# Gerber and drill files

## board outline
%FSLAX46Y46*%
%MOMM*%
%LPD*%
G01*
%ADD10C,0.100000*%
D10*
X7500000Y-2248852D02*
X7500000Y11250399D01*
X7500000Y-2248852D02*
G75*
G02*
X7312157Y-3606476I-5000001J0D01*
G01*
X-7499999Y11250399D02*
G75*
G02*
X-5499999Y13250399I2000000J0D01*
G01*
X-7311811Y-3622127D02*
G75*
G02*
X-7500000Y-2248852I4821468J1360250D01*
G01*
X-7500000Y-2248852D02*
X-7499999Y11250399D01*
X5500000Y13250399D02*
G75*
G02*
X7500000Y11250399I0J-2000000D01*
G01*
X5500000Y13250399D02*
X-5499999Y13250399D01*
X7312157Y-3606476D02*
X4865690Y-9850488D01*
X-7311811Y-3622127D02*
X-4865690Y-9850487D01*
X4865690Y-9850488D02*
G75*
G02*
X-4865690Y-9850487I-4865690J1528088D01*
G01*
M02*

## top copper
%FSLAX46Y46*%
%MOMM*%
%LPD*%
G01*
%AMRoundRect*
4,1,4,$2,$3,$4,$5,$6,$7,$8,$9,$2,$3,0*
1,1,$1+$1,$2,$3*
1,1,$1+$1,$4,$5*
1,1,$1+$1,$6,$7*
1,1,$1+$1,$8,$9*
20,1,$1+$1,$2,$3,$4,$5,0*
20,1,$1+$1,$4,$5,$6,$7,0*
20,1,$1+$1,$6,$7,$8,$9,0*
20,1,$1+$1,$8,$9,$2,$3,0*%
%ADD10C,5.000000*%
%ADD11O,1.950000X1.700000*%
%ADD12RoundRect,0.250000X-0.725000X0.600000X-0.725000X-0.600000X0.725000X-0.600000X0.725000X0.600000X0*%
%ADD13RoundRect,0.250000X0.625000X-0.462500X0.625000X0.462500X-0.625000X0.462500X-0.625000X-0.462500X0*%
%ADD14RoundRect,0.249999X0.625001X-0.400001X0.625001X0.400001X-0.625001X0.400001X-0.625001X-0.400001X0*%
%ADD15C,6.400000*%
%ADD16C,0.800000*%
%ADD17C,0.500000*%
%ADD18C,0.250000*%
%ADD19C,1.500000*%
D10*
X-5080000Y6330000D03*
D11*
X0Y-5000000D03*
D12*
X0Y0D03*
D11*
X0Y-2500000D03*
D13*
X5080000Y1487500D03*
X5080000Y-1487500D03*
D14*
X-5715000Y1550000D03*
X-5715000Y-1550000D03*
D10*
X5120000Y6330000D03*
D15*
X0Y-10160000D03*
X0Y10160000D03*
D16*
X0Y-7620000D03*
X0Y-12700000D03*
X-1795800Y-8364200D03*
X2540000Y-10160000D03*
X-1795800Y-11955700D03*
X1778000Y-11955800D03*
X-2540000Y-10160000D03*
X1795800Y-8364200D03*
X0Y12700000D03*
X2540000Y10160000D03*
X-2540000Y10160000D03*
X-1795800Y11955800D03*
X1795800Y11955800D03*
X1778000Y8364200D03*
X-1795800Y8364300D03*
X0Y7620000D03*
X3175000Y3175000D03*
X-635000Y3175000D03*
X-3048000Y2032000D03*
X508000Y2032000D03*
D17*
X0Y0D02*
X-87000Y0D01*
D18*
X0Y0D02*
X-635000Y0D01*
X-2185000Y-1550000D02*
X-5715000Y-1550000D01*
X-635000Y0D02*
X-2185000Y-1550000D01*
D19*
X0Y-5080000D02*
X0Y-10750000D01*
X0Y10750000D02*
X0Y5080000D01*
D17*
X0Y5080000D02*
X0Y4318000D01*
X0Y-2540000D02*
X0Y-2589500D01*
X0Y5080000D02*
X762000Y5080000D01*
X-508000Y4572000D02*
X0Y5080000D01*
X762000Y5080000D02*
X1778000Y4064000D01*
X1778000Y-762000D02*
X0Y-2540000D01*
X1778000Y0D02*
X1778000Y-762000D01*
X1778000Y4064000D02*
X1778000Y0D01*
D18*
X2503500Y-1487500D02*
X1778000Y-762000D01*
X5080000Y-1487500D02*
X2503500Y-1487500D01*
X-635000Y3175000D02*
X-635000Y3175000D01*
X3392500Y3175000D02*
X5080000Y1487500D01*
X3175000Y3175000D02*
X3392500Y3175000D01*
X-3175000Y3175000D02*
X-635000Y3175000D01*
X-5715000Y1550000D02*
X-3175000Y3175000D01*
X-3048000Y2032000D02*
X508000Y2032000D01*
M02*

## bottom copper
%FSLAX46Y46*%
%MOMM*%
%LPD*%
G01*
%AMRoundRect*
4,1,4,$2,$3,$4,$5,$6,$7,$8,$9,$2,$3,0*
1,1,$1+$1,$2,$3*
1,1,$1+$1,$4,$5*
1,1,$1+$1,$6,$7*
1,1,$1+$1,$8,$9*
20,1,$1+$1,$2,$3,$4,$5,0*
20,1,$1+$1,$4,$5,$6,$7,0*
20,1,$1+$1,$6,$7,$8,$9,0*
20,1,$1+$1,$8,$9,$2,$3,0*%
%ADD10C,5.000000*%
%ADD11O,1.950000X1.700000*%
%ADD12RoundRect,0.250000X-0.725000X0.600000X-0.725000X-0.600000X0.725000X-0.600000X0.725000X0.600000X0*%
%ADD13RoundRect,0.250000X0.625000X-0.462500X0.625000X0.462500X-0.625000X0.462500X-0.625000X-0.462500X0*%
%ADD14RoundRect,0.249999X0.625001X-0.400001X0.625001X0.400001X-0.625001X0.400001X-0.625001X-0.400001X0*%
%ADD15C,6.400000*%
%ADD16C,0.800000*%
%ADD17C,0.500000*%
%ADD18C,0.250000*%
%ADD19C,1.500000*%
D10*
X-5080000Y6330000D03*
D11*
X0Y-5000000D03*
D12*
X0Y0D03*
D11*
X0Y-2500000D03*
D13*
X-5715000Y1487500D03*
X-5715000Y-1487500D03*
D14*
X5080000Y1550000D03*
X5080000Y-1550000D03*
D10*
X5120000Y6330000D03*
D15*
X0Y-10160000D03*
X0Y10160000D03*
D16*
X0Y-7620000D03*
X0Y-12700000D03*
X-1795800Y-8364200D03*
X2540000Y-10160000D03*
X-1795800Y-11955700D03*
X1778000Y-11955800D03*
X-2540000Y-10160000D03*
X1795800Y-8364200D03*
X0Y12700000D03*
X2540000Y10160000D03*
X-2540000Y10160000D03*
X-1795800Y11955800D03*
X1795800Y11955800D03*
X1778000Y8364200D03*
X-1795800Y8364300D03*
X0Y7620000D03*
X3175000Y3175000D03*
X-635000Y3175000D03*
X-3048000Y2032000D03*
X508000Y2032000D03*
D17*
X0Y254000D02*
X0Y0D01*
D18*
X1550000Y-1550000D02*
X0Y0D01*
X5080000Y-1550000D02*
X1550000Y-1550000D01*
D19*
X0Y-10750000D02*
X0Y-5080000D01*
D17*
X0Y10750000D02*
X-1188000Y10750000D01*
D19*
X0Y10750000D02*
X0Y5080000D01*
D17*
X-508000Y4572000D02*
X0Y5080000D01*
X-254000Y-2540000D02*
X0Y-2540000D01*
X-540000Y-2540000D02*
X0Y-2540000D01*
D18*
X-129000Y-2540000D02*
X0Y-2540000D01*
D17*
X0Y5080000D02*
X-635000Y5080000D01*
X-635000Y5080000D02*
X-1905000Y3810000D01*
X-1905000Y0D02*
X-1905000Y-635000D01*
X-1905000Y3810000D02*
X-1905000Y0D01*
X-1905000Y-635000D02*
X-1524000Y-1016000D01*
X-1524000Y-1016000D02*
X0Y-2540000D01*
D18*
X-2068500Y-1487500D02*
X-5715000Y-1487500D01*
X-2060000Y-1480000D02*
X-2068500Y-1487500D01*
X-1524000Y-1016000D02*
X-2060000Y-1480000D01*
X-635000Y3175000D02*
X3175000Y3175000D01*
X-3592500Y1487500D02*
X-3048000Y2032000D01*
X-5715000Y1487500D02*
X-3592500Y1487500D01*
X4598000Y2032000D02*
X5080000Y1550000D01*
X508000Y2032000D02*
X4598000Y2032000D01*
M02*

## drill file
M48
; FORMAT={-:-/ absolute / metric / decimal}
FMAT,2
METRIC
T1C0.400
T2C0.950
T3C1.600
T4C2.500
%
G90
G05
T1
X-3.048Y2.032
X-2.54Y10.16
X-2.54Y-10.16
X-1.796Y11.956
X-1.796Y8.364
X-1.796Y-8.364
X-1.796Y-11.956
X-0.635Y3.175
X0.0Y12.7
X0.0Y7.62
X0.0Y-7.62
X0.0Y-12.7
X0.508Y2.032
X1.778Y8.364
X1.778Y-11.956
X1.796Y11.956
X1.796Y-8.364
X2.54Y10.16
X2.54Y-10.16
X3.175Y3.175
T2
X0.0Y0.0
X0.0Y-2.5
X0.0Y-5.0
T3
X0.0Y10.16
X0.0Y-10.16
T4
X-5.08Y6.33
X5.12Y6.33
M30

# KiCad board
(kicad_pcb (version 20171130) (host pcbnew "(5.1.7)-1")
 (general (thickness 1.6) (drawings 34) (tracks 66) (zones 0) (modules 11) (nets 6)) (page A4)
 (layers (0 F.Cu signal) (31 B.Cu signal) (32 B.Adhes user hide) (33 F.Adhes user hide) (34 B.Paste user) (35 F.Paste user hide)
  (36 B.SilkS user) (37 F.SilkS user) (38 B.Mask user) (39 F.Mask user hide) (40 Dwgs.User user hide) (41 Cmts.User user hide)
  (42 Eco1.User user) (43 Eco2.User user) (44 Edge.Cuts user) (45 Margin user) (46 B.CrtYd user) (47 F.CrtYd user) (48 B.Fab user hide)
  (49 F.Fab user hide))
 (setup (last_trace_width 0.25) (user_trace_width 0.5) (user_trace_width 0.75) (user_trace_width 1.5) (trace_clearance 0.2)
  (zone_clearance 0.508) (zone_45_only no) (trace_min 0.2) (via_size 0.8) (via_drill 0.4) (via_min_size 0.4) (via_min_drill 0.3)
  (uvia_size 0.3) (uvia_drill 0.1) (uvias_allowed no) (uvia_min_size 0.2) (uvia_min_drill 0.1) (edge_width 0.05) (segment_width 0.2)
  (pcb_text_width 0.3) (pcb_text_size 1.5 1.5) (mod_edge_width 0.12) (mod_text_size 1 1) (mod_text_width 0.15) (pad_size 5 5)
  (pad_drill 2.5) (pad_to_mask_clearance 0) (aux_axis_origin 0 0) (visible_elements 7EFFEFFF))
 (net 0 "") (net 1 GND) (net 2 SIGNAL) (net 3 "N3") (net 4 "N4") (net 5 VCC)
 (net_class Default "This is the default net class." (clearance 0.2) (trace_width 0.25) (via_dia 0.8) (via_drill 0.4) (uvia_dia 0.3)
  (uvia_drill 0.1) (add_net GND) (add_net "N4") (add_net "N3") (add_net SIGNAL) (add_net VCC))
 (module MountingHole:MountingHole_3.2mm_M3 (layer F.Cu) (at -5.08 -6.33)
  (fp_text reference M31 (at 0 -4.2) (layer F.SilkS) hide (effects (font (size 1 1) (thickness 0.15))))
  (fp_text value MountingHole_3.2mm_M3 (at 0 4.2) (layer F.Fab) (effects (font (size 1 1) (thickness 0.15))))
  (pad "" np_thru_hole circle (at 0 0) (size 5 5) (drill 2.5) (layers *.Cu *.Mask)))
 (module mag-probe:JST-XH (layer F.Cu) (at 0 0 270)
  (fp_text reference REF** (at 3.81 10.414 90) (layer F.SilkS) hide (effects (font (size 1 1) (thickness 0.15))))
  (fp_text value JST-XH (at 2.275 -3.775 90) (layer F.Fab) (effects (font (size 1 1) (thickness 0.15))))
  (pad 3 thru_hole oval (at 5 0 270) (size 1.7 1.95) (drill 0.95) (layers *.Cu *.Mask) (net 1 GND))
  (pad 1 thru_hole roundrect (at 0 0 270) (size 1.7 1.95) (drill 0.95) (layers *.Cu *.Mask) (roundrect_rratio 0.1470588235294118))
  (pad 2 thru_hole oval (at 2.5 0 270) (size 1.7 1.95) (drill 0.95) (layers *.Cu *.Mask) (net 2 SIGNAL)))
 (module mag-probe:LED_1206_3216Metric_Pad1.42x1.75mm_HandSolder (layer B.Cu) (at -5.715 0 90)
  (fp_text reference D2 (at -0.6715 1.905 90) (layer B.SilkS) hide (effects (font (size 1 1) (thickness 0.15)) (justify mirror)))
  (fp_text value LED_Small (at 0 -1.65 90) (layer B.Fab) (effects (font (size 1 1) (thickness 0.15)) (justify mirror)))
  (pad 2 smd roundrect (at 1.4875 0 90) (size 1.425 1.75) (layers B.Cu B.Paste B.Mask) (roundrect_rratio 0.1754385964912281) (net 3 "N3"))
  (pad 1 smd roundrect (at -1.4875 0 90) (size 1.425 1.75) (layers B.Cu B.Paste B.Mask) (roundrect_rratio 0.1754385964912281) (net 2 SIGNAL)))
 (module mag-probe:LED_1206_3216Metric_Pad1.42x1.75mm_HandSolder (layer F.Cu) (at 5.08 0 90)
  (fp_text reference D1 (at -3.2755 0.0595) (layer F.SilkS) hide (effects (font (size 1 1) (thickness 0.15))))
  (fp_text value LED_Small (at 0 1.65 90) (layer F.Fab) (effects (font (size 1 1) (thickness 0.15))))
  (pad 2 smd roundrect (at 1.4875 0 90) (size 1.425 1.75) (layers F.Cu F.Paste F.Mask) (roundrect_rratio 0.1754385964912281) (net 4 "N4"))
  (pad 1 smd roundrect (at -1.4875 0 90) (size 1.425 1.75) (layers F.Cu F.Paste F.Mask) (roundrect_rratio 0.1754385964912281) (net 2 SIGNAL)))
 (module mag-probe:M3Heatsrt (layer F.Cu) (at -5.08 -6.33)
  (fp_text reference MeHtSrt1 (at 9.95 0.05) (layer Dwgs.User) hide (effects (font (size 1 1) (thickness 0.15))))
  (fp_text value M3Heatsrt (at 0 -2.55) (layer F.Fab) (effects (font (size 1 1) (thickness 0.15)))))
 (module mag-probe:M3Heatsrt (layer F.Cu) (at 5.08 -6.33)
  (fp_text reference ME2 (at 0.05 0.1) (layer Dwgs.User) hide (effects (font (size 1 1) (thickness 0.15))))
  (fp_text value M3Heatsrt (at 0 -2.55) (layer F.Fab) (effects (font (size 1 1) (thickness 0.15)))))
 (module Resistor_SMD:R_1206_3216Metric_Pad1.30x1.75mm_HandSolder (layer F.Cu) (at -5.715 0 90)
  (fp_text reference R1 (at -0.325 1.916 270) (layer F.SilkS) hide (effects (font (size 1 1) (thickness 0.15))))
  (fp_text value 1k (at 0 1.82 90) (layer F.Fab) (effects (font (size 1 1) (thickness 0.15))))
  (pad 2 smd roundrect (at 1.55 0 90) (size 1.3 1.75) (layers F.Cu F.Paste F.Mask) (roundrect_rratio 0.1923069230769231) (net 4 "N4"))
  (pad 1 smd roundrect (at -1.55 0 90) (size 1.3 1.75) (layers F.Cu F.Paste F.Mask) (roundrect_rratio 0.1923069230769231) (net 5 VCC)))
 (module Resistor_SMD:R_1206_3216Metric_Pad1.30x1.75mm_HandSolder (layer B.Cu) (at 5.08 0 90)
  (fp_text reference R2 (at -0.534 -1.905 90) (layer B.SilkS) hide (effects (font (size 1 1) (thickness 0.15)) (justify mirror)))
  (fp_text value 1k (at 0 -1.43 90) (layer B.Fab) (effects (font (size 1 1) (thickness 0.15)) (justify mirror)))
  (pad 2 smd roundrect (at 1.55 0 90) (size 1.3 1.75) (layers B.Cu B.Paste B.Mask) (roundrect_rratio 0.1923069230769231) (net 3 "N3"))
  (pad 1 smd roundrect (at -1.55 0 90) (size 1.3 1.75) (layers B.Cu B.Paste B.Mask) (roundrect_rratio 0.1923069230769231) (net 5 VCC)))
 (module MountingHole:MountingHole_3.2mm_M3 (layer F.Cu) (at 5.08 -6.33)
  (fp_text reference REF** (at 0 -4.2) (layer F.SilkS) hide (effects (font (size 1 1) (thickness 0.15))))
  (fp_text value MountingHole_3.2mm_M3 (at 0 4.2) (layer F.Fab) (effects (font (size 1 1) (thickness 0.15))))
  (pad "" np_thru_hole circle (at 0.04 0) (size 5 5) (drill 2.5) (layers *.Cu *.Mask)))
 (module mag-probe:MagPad (layer B.Cu) (at 0 10.16)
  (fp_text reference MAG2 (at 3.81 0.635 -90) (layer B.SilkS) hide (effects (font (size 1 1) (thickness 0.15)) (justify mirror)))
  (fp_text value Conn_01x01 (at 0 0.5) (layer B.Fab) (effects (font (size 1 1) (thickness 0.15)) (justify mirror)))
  (pad 1 thru_hole circle (at 0 0) (size 6.4 6.4) (drill 1.6) (layers *.Cu *.Mask) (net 1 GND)))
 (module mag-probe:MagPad (layer B.Cu) (at 0 -10.16)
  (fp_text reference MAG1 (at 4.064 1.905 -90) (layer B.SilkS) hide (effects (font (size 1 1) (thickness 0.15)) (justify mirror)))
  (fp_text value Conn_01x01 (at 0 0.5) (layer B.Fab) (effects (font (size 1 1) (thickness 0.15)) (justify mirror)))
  (pad 1 thru_hole circle (at 0 0) (size 6.4 6.4) (drill 1.6) (layers *.Cu *.Mask) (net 2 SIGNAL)))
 (gr_line (start 7.5 2.248852) (end 7.5 -11.250399) (layer Edge.Cuts) (width 0.1))
 (gr_arc (start 2.499999 2.248852) (end 7.312157 3.606476) (angle -15.75501346) (layer Edge.Cuts) (width 0.1))
 (gr_arc (start -5.499999 -11.250399) (end -5.499999 -13.250399) (angle -90) (layer Edge.Cuts) (width 0.1))
 (gr_arc (start -2.490343 2.261877) (end -7.5 2.248852) (angle -15.90398022) (layer Edge.Cuts) (width 0.1))
 (gr_line (start -7.5 2.248852) (end -7.499999 -11.250399) (layer Edge.Cuts) (width 0.1))
 (gr_arc (start 5.5 -11.250399) (end 7.5 -11.250399) (angle -90) (layer Edge.Cuts) (width 0.1))
 (gr_line (start 5.5 -13.250399) (end -5.499999 -13.250399) (layer Edge.Cuts) (width 0.1))
 (gr_line (start 7.312157 3.606476) (end 4.86569 9.850488) (layer Edge.Cuts) (width 0.1))
 (gr_line (start -7.311811 3.622127) (end -4.86569 9.850487) (layer Edge.Cuts) (width 0.1))
 (gr_arc (start 0 8.3224) (end -4.86569 9.850487) (angle -145.1298326) (layer Edge.Cuts) (width 0.1))
 (segment (start 0 -0.254) (end 0 0) (width 0.5) (layer B.Cu) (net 5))
 (segment (start 0 0) (end -0.087 0) (width 0.5) (layer F.Cu) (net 5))
 (segment (start 0 0) (end -0.635 0) (width 0.25) (layer F.Cu) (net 5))
 (segment (start -2.185 1.55) (end -5.715 1.55) (width 0.25) (layer F.Cu) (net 5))
 (segment (start -0.635 0) (end -2.185 1.55) (width 0.25) (layer F.Cu) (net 5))
 (segment (start 1.55 1.55) (end 0 0) (width 0.25) (layer B.Cu) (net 5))
 (segment (start 5.08 1.55) (end 1.55 1.55) (width 0.25) (layer B.Cu) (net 5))
 (segment (start 0 10.75) (end 0 5.08) (width 1.5) (layer B.Cu) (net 1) (status 30))
 (segment (start 0 5.08) (end 0 10.75) (width 1.5) (layer F.Cu) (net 1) (status 30))
 (via (at 0 7.62) (size 0.8) (drill 0.4) (layers F.Cu B.Cu) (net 1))
 (via (at 0 12.7) (size 0.8) (drill 0.4) (layers F.Cu B.Cu) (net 1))
 (via (at -1.7958 8.3642) (size 0.8) (drill 0.4) (layers F.Cu B.Cu) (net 1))
 (via (at 2.54 10.16) (size 0.8) (drill 0.4) (layers F.Cu B.Cu) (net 1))
 (via (at -1.7958 11.9557) (size 0.8) (drill 0.4) (layers F.Cu B.Cu) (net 1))
 (via (at 1.778 11.9558) (size 0.8) (drill 0.4) (layers F.Cu B.Cu) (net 1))
 (via (at -2.54 10.16) (size 0.8) (drill 0.4) (layers F.Cu B.Cu) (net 1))
 (via (at 1.7958 8.3642) (size 0.8) (drill 0.4) (layers F.Cu B.Cu) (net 1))
 (via (at 0 -12.7) (size 0.8) (drill 0.4) (layers F.Cu B.Cu) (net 2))
 (via (at 2.54 -10.16) (size 0.8) (drill 0.4) (layers F.Cu B.Cu) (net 2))
 (via (at -2.54 -10.16) (size 0.8) (drill 0.4) (layers F.Cu B.Cu) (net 2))
 (via (at -1.7958 -11.9558) (size 0.8) (drill 0.4) (layers F.Cu B.Cu) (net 2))
 (via (at 1.7958 -11.9558) (size 0.8) (drill 0.4) (layers F.Cu B.Cu) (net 2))
 (via (at 1.778 -8.3642) (size 0.8) (drill 0.4) (layers F.Cu B.Cu) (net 2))
 (via (at -1.7958 -8.3643) (size 0.8) (drill 0.4) (layers F.Cu B.Cu) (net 2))
 (via (at 0 -7.62) (size 0.8) (drill 0.4) (layers F.Cu B.Cu) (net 2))
 (segment (start 0 -10.75) (end -1.188 -10.75) (width 0.5) (layer B.Cu) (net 2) (status 30))
 (segment (start 0 -10.75) (end 0 -5.08) (width 1.5) (layer B.Cu) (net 2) (status 30))
 (segment (start -0.508 -4.572) (end 0 -5.08) (width 0.5) (layer B.Cu) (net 2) (status 30))
 (segment (start 0 -10.75) (end 0 -5.08) (width 1.5) (layer F.Cu) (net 2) (status 30))
 (segment (start -0.254 2.54) (end 0 2.54) (width 0.5) (layer B.Cu) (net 2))
 (segment (start 0 -5.08) (end 0 -4.318) (width 0.5) (layer F.Cu) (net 2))
 (segment (start 0 2.54) (end 0 2.5895) (width 0.5) (layer F.Cu) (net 2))
 (segment (start -0.54 2.54) (end 0 2.54) (width 0.5) (layer B.Cu) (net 2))
 (segment (start -0.129 2.54) (end 0 2.54) (width 0.25) (layer B.Cu) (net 2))
 (segment (start 0 -5.08) (end 0.762 -5.08) (width 0.5) (layer F.Cu) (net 2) (status 30))
 (segment (start -0.508 -4.572) (end 0 -5.08) (width 0.5) (layer F.Cu) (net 2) (status 30))
 (segment (start 0 -5.08) (end -0.635 -5.08) (width 0.5) (layer B.Cu) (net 2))
 (segment (start -0.635 -5.08) (end -1.905 -3.81) (width 0.5) (layer B.Cu) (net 2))
 (segment (start 0.762 -5.08) (end 1.778 -4.064) (width 0.5) (layer F.Cu) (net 2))
 (segment (start 1.778 0.762) (end 0 2.54) (width 0.5) (layer F.Cu) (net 2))
 (segment (start 1.778 0) (end 1.778 0.762) (width 0.5) (layer F.Cu) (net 2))
 (segment (start 1.778 -4.064) (end 1.778 0) (width 0.5) (layer F.Cu) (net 2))
 (segment (start -1.905 0) (end -1.905 0.635) (width 0.5) (layer B.Cu) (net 2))
 (segment (start -1.905 -3.81) (end -1.905 0) (width 0.5) (layer B.Cu) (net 2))
 (segment (start 2.5035 1.4875) (end 1.778 0.762) (width 0.25) (layer F.Cu) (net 2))
 (segment (start 5.08 1.4875) (end 2.5035 1.4875) (width 0.25) (layer F.Cu) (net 2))
 (segment (start -1.905 0.635) (end -1.524 1.016) (width 0.5) (layer B.Cu) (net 2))
 (segment (start -1.524 1.016) (end 0 2.54) (width 0.5) (layer B.Cu) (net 2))
 (segment (start -2.0685 1.4875) (end -5.715 1.4875) (width 0.25) (layer B.Cu) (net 2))
 (segment (start -2.06 1.48) (end -2.0685 1.4875) (width 0.25) (layer B.Cu) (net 2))
 (segment (start -1.524 1.016) (end -2.06 1.48) (width 0.25) (layer B.Cu) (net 2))
 (via (at 3.175 -3.175) (size 0.8) (drill 0.4) (layers F.Cu B.Cu) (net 4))
 (segment (start -0.635 -3.175) (end -0.635 -3.175) (width 0.25) (layer F.Cu) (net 4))
 (via (at -0.635 -3.175) (size 0.8) (drill 0.4) (layers F.Cu B.Cu) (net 4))
 (segment (start -0.635 -3.175) (end 3.175 -3.175) (width 0.25) (layer B.Cu) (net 4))
 (segment (start 3.3925 -3.175) (end 5.08 -1.4875) (width 0.25) (layer F.Cu) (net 4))
 (segment (start 3.175 -3.175) (end 3.3925 -3.175) (width 0.25) (layer F.Cu) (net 4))
 (segment (start -3.175 -3.175) (end -0.635 -3.175) (width 0.25) (layer F.Cu) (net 4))
 (segment (start -5.715 -1.55) (end -3.175 -3.175) (width 0.25) (layer F.Cu) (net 4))
 (via (at -3.048 -2.032) (size 0.8) (drill 0.4) (layers F.Cu B.Cu) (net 3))
 (via (at 0.508 -2.032) (size 0.8) (drill 0.4) (layers F.Cu B.Cu) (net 3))
 (segment (start -3.5925 -1.4875) (end -3.048 -2.032) (width 0.25) (layer B.Cu) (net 3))
 (segment (start -5.715 -1.4875) (end -3.5925 -1.4875) (width 0.25) (layer B.Cu) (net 3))
 (segment (start 4.598 -2.032) (end 5.08 -1.55) (width 0.25) (layer B.Cu) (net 3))
 (segment (start 0.508 -2.032) (end 4.598 -2.032) (width 0.25) (layer B.Cu) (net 3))
 (segment (start -3.048 -2.032) (end 0.508 -2.032) (width 0.25) (layer F.Cu) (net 3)))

